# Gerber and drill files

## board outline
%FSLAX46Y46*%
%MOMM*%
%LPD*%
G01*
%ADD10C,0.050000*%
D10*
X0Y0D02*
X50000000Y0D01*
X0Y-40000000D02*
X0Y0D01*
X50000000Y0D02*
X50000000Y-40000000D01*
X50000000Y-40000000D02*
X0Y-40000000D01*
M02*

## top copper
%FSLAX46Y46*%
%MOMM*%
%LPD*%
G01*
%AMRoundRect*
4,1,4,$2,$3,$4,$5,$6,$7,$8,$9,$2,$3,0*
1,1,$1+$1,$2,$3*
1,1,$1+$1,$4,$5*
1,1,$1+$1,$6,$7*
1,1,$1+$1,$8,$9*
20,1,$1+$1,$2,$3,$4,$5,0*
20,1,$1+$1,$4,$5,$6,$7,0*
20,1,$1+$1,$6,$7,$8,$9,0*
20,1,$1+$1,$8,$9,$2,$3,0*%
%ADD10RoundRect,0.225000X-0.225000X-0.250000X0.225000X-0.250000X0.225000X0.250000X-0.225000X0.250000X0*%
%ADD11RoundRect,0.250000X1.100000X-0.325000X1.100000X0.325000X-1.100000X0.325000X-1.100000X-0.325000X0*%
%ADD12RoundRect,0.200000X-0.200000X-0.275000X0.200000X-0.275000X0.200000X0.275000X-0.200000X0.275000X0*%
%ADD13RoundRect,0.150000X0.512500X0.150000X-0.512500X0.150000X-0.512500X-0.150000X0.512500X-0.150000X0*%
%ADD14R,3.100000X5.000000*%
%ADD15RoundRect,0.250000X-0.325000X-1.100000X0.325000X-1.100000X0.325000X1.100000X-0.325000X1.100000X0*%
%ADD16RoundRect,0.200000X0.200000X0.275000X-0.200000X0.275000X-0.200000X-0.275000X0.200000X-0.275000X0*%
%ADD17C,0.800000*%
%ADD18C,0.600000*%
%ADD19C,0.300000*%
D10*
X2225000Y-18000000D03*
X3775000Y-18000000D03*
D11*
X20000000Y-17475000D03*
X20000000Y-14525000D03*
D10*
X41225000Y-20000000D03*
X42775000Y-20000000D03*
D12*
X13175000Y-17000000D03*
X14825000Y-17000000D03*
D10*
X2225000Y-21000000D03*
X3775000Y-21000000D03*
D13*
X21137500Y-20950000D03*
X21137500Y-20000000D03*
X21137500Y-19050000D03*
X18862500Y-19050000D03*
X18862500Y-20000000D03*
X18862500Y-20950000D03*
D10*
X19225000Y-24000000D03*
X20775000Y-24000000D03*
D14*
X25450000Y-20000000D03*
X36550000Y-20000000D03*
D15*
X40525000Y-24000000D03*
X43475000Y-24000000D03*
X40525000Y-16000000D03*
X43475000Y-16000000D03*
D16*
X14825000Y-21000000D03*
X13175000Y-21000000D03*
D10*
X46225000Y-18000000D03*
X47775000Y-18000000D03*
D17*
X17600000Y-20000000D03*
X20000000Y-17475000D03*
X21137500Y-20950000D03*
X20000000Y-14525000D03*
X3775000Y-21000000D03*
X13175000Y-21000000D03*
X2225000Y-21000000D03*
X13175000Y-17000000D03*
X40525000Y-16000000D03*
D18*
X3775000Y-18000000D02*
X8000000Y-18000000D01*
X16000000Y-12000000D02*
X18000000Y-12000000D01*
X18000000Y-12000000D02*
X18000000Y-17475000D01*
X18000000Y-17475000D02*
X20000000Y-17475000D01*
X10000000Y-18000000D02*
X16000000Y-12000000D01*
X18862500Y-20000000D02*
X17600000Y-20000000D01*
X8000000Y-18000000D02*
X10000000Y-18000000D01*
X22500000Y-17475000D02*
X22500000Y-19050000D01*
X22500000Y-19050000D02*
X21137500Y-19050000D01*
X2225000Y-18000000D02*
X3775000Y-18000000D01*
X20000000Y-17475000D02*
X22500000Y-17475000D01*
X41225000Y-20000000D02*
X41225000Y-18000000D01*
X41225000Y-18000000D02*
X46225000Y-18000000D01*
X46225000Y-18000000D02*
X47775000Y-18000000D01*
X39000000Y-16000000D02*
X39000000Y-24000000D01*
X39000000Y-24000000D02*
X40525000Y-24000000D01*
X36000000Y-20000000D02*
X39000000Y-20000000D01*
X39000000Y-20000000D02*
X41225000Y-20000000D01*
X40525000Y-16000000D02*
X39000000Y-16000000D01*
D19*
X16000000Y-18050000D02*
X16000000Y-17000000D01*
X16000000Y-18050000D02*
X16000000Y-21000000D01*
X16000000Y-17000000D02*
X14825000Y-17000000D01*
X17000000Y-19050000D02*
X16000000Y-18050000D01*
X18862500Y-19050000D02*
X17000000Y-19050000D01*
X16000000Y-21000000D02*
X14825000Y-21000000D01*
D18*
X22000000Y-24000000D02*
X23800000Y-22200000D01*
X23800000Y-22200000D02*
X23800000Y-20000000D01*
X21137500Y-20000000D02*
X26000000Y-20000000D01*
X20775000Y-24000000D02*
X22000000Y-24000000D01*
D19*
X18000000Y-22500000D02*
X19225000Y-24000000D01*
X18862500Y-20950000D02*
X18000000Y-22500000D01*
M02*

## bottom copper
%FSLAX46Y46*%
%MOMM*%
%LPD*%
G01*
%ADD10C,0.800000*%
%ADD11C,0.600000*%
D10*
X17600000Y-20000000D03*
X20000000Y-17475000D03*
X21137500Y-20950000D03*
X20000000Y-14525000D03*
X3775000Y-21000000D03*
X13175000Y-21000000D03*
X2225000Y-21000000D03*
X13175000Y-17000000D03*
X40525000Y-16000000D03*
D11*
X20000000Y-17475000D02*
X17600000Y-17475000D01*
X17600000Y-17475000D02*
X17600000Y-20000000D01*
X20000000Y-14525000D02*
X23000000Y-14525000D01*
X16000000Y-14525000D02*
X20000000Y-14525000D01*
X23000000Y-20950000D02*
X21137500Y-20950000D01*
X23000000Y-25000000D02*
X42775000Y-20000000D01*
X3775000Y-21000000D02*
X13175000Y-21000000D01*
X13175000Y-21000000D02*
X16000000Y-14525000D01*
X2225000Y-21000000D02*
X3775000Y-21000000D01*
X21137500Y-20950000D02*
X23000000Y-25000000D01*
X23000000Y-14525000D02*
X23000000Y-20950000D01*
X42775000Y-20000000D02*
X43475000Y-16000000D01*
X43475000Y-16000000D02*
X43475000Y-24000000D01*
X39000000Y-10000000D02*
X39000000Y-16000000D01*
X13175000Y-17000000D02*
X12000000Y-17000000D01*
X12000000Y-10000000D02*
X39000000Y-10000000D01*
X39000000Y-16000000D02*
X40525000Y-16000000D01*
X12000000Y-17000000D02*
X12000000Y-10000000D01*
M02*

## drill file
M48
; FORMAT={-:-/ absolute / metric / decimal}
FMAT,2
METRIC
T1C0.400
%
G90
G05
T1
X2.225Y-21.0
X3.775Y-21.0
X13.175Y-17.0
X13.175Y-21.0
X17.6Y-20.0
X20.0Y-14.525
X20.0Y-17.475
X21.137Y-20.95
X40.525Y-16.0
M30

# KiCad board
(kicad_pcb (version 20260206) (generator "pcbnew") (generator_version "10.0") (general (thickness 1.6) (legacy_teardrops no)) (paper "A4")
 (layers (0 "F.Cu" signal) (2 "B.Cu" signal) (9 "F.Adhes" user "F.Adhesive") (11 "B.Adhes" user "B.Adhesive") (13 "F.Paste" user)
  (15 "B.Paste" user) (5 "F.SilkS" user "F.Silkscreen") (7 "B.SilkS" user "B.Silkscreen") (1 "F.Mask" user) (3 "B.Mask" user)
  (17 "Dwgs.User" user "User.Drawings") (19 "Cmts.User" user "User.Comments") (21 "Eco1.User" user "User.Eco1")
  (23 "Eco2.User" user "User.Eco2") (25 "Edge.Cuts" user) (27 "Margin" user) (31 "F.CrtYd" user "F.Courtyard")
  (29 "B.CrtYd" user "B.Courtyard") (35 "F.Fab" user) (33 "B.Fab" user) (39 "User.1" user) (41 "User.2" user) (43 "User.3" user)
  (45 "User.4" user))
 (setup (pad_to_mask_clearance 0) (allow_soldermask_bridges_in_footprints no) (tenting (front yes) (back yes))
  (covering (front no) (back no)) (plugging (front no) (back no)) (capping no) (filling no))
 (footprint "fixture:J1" (layer "F.Cu") (at 3 18)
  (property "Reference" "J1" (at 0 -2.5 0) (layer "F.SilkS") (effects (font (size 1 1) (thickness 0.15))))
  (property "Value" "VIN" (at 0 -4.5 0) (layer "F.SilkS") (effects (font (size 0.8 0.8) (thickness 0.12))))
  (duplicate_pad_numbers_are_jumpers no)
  (pad "1" smd roundrect (at -0.775 0) (size 0.9 0.95) (layers "F.Cu" "F.Mask" "F.Paste") (roundrect_rratio 0.25) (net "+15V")
   (thermal_bridge_angle 45))
  (pad "2" smd roundrect (at 0.775 0) (size 0.9 0.95) (layers "F.Cu" "F.Mask" "F.Paste") (roundrect_rratio 0.25) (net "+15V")
   (thermal_bridge_angle 45)))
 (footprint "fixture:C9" (layer "F.Cu") (at 20 16 90)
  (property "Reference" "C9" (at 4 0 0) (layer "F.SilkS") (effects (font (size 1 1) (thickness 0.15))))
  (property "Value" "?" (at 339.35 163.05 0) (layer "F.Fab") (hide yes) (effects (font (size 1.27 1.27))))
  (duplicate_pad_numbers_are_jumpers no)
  (pad "1" smd roundrect (at -1.475 0 90) (size 1.15 2.7) (layers "F.Cu" "F.Mask" "F.Paste") (roundrect_rratio 0.217391) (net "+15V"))
  (pad "2" smd roundrect (at 1.475 0 90) (size 1.15 2.7) (layers "F.Cu" "F.Mask" "F.Paste") (roundrect_rratio 0.217391) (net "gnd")))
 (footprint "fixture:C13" (layer "F.Cu") (at 42 20)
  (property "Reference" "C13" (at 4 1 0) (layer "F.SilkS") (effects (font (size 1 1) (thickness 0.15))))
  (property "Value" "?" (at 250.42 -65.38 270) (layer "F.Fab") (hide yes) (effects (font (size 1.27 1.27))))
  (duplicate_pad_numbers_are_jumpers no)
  (pad "1" smd roundrect (at -0.775 0) (size 0.9 0.95) (layers "F.Cu" "F.Mask" "F.Paste") (roundrect_rratio 0.25) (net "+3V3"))
  (pad "2" smd roundrect (at 0.775 0) (size 0.9 0.95) (layers "F.Cu" "F.Mask" "F.Paste") (roundrect_rratio 0.25) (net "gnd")))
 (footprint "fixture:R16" (layer "F.Cu") (at 14 17)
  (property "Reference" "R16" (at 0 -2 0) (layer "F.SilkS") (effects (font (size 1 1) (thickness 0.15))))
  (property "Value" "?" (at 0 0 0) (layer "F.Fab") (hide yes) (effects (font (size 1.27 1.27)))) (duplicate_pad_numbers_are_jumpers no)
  (pad "1" smd roundrect (at -0.825 0) (size 0.8 0.95) (layers "F.Cu" "F.Mask" "F.Paste") (roundrect_rratio 0.25) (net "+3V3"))
  (pad "2" smd roundrect (at 0.825 0) (size 0.8 0.95) (layers "F.Cu" "F.Mask" "F.Paste") (roundrect_rratio 0.25) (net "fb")))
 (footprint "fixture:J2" (layer "F.Cu") (at 3 21)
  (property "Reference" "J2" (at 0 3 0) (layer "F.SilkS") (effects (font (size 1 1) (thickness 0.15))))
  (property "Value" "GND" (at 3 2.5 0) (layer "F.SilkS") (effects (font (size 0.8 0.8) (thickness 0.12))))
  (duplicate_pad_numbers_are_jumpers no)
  (pad "1" smd roundrect (at -0.775 0) (size 0.9 0.95) (layers "F.Cu" "F.Mask" "F.Paste") (roundrect_rratio 0.25) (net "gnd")
   (thermal_bridge_angle 45))
  (pad "2" smd roundrect (at 0.775 0) (size 0.9 0.95) (layers "F.Cu" "F.Mask" "F.Paste") (roundrect_rratio 0.25) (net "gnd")
   (thermal_bridge_angle 45)))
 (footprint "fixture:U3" (layer "F.Cu") (at 20 20 180)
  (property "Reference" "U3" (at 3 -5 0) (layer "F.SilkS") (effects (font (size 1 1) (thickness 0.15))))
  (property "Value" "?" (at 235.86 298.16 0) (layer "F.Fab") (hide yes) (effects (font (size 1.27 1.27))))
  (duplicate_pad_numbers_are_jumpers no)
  (pad "1" smd roundrect (at -1.1375 -0.95 180) (size 1.325 0.6) (layers "F.Cu" "F.Mask" "F.Paste") (roundrect_rratio 0.25) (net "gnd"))
  (pad "2" smd roundrect (at -1.1375 0 180) (size 1.325 0.6) (layers "F.Cu" "F.Mask" "F.Paste") (roundrect_rratio 0.25) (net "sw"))
  (pad "3" smd roundrect (at -1.1375 0.95 180) (size 1.325 0.6) (layers "F.Cu" "F.Mask" "F.Paste") (roundrect_rratio 0.25) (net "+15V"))
  (pad "4" smd roundrect (at 1.1375 0.95 180) (size 1.325 0.6) (layers "F.Cu" "F.Mask" "F.Paste") (roundrect_rratio 0.25) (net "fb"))
  (pad "5" smd roundrect (at 1.1375 0 180) (size 1.325 0.6) (layers "F.Cu" "F.Mask" "F.Paste") (roundrect_rratio 0.25) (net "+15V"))
  (pad "6" smd roundrect (at 1.1375 -0.95 180) (size 1.325 0.6) (layers "F.Cu" "F.Mask" "F.Paste") (roundrect_rratio 0.25) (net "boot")))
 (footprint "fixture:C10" (layer "F.Cu") (at 20 24)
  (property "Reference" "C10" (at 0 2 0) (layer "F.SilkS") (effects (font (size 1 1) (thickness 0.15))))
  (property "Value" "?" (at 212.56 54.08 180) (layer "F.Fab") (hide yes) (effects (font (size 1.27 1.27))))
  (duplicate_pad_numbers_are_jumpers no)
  (pad "1" smd roundrect (at -0.775 0) (size 0.9 0.95) (layers "F.Cu" "F.Mask" "F.Paste") (roundrect_rratio 0.25) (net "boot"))
  (pad "2" smd roundrect (at 0.775 0) (size 0.9 0.95) (layers "F.Cu" "F.Mask" "F.Paste") (roundrect_rratio 0.25) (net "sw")))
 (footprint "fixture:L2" (layer "F.Cu") (at 31 20)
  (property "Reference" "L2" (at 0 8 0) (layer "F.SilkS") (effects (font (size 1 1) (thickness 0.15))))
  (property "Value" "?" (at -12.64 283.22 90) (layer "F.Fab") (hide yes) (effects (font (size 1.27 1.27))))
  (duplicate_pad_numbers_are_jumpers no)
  (pad "1" smd rect (at -5.55 0) (size 3.1 5) (layers "F.Cu" "F.Mask" "F.Paste") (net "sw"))
  (pad "2" smd rect (at 5.55 0) (size 3.1 5) (layers "F.Cu" "F.Mask" "F.Paste") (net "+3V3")))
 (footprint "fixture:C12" (layer "F.Cu") (at 42 24)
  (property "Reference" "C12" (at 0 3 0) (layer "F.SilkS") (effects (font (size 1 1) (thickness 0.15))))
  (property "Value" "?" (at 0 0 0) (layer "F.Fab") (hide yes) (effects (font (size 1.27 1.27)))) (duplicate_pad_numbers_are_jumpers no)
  (pad "1" smd roundrect (at -1.475 0) (size 1.15 2.7) (layers "F.Cu" "F.Mask" "F.Paste") (roundrect_rratio 0.217391) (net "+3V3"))
  (pad "2" smd roundrect (at 1.475 0) (size 1.15 2.7) (layers "F.Cu" "F.Mask" "F.Paste") (roundrect_rratio 0.217391) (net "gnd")))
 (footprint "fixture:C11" (layer "F.Cu") (at 42 16)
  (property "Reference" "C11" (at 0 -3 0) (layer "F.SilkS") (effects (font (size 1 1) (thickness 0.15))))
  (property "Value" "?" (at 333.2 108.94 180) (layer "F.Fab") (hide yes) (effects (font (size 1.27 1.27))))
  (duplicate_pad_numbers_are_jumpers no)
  (pad "1" smd roundrect (at -1.475 0) (size 1.15 2.7) (layers "F.Cu" "F.Mask" "F.Paste") (roundrect_rratio 0.217391) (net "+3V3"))
  (pad "2" smd roundrect (at 1.475 0) (size 1.15 2.7) (layers "F.Cu" "F.Mask" "F.Paste") (roundrect_rratio 0.217391) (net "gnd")))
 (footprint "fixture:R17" (layer "F.Cu") (at 14 21 180)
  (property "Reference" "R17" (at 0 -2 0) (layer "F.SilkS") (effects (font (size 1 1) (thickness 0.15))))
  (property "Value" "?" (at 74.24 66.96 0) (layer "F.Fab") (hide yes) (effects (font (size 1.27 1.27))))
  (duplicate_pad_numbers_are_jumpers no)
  (pad "1" smd roundrect (at -0.825 0 180) (size 0.8 0.95) (layers "F.Cu" "F.Mask" "F.Paste") (roundrect_rratio 0.25) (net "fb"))
  (pad "2" smd roundrect (at 0.825 0 180) (size 0.8 0.95) (layers "F.Cu" "F.Mask" "F.Paste") (roundrect_rratio 0.25) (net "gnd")))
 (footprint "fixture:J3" (layer "F.Cu") (at 47 18)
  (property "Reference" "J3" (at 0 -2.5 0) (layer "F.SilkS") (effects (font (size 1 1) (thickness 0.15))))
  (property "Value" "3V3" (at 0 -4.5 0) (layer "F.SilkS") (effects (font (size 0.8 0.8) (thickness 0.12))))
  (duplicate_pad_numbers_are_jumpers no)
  (pad "1" smd roundrect (at -0.775 0) (size 0.9 0.95) (layers "F.Cu" "F.Mask" "F.Paste") (roundrect_rratio 0.25) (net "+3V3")
   (thermal_bridge_angle 45))
  (pad "2" smd roundrect (at 0.775 0) (size 0.9 0.95) (layers "F.Cu" "F.Mask" "F.Paste") (roundrect_rratio 0.25) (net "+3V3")
   (thermal_bridge_angle 45)))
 (gr_line (start 0 0) (end 50 0) (stroke (width 0.05) (type default)) (layer "Edge.Cuts"))
 (gr_line (start 0 40) (end 0 0) (stroke (width 0.05) (type default)) (layer "Edge.Cuts"))
 (gr_line (start 50 0) (end 50 40) (stroke (width 0.05) (type default)) (layer "Edge.Cuts"))
 (gr_line (start 50 40) (end 0 40) (stroke (width 0.05) (type default)) (layer "Edge.Cuts"))
 (segment (start 3.775 18) (end 8 18) (width 0.6) (layer "F.Cu") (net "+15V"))
 (segment (start 16 12) (end 18 12) (width 0.6) (layer "F.Cu") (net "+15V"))
 (segment (start 18 12) (end 18 17.475) (width 0.6) (layer "F.Cu") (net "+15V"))
 (segment (start 18 17.475) (end 20 17.475) (width 0.6) (layer "F.Cu") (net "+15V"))
 (segment (start 10 18) (end 16 12) (width 0.6) (layer "F.Cu") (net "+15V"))
 (segment (start 18.8625 20) (end 17.6 20) (width 0.6) (layer "F.Cu") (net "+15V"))
 (segment (start 8 18) (end 10 18) (width 0.6) (layer "F.Cu") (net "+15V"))
 (segment (start 22.5 17.475) (end 22.5 19.05) (width 0.6) (layer "F.Cu") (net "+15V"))
 (segment (start 22.5 19.05) (end 21.1375 19.05) (width 0.6) (layer "F.Cu") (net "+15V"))
 (segment (start 2.225 18) (end 3.775 18) (width 0.6) (layer "F.Cu") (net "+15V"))
 (segment (start 20 17.475) (end 22.5 17.475) (width 0.6) (layer "F.Cu") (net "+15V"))
 (via (at 17.6 20) (size 0.8) (drill 0.4) (layers "F.Cu" "B.Cu") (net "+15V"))
 (via (at 20 17.475) (size 0.8) (drill 0.4) (layers "F.Cu" "B.Cu") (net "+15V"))
 (segment (start 20 17.475) (end 17.6 17.475) (width 0.6) (layer "B.Cu") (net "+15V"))
 (segment (start 17.6 17.475) (end 17.6 20) (width 0.6) (layer "B.Cu") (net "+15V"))
 (via (at 21.1375 20.95) (size 0.8) (drill 0.4) (layers "F.Cu" "B.Cu") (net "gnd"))
 (via (at 20 14.525) (size 0.8) (drill 0.4) (layers "F.Cu" "B.Cu") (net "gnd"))
 (via (at 3.775 21) (size 0.8) (drill 0.4) (layers "F.Cu" "B.Cu") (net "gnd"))
 (via (at 13.175 21) (size 0.8) (drill 0.4) (layers "F.Cu" "B.Cu") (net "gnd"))
 (via (at 2.225 21) (size 0.8) (drill 0.4) (layers "F.Cu" "B.Cu") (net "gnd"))
 (segment (start 20 14.525) (end 23 14.525) (width 0.6) (layer "B.Cu") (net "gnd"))
 (segment (start 16 14.525) (end 20 14.525) (width 0.6) (layer "B.Cu") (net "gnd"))
 (segment (start 23 20.95) (end 21.1375 20.95) (width 0.6) (layer "B.Cu") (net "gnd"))
 (segment (start 23 25) (end 42.775 20) (width 0.6) (layer "B.Cu") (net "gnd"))
 (segment (start 3.775 21) (end 13.175 21) (width 0.6) (layer "B.Cu") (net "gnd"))
 (segment (start 13.175 21) (end 16 14.525) (width 0.6) (layer "B.Cu") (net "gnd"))
 (segment (start 2.225 21) (end 3.775 21) (width 0.6) (layer "B.Cu") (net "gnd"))
 (segment (start 21.1375 20.95) (end 23 25) (width 0.6) (layer "B.Cu") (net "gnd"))
 (segment (start 23 14.525) (end 23 20.95) (width 0.6) (layer "B.Cu") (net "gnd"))
 (segment (start 42.775 20) (end 43.475 16) (width 0.6) (layer "B.Cu") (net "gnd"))
 (segment (start 43.475 16) (end 43.475 24) (width 0.6) (layer "B.Cu") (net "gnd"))
 (segment (start 41.225 20) (end 41.225 18) (width 0.6) (layer "F.Cu") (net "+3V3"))
 (segment (start 41.225 18) (end 46.225 18) (width 0.6) (layer "F.Cu") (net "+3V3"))
 (segment (start 46.225 18) (end 47.775 18) (width 0.6) (layer "F.Cu") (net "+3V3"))
 (segment (start 39 16) (end 39 24) (width 0.6) (layer "F.Cu") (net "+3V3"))
 (segment (start 39 24) (end 40.525 24) (width 0.6) (layer "F.Cu") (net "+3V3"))
 (segment (start 36 20) (end 39 20) (width 0.6) (layer "F.Cu") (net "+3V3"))
 (segment (start 39 20) (end 41.225 20) (width 0.6) (layer "F.Cu") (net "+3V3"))
 (segment (start 40.525 16) (end 39 16) (width 0.6) (layer "F.Cu") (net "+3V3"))
 (via (at 13.175 17) (size 0.8) (drill 0.4) (layers "F.Cu" "B.Cu") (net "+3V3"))
 (via (at 40.525 16) (size 0.8) (drill 0.4) (layers "F.Cu" "B.Cu") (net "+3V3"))
 (segment (start 39 10) (end 39 16) (width 0.6) (layer "B.Cu") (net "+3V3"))
 (segment (start 13.175 17) (end 12 17) (width 0.6) (layer "B.Cu") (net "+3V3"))
 (segment (start 12 10) (end 39 10) (width 0.6) (layer "B.Cu") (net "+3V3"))
 (segment (start 39 16) (end 40.525 16) (width 0.6) (layer "B.Cu") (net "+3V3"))
 (segment (start 12 17) (end 12 10) (width 0.6) (layer "B.Cu") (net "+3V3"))
 (segment (start 16 18.05) (end 16 17) (width 0.3) (layer "F.Cu") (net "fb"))
 (segment (start 16 18.05) (end 16 21) (width 0.3) (layer "F.Cu") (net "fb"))
 (segment (start 16 17) (end 14.825 17) (width 0.3) (layer "F.Cu") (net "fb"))
 (segment (start 17 19.05) (end 16 18.05) (width 0.3) (layer "F.Cu") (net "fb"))
 (segment (start 18.8625 19.05) (end 17 19.05) (width 0.3) (layer "F.Cu") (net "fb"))
 (segment (start 16 21) (end 14.825 21) (width 0.3) (layer "F.Cu") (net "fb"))
 (segment (start 22 24) (end 23.8 22.2) (width 0.6) (layer "F.Cu") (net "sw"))
 (segment (start 23.8 22.2) (end 23.8 20) (width 0.6) (layer "F.Cu") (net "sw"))
 (segment (start 21.1375 20) (end 26 20) (width 0.6) (layer "F.Cu") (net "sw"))
 (segment (start 20.775 24) (end 22 24) (width 0.6) (layer "F.Cu") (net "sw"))
 (segment (start 18 22.5) (end 19.225 24) (width 0.3) (layer "F.Cu") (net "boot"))
 (segment (start 18.8625 20.95) (end 18 22.5) (width 0.3) (layer "F.Cu") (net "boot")))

